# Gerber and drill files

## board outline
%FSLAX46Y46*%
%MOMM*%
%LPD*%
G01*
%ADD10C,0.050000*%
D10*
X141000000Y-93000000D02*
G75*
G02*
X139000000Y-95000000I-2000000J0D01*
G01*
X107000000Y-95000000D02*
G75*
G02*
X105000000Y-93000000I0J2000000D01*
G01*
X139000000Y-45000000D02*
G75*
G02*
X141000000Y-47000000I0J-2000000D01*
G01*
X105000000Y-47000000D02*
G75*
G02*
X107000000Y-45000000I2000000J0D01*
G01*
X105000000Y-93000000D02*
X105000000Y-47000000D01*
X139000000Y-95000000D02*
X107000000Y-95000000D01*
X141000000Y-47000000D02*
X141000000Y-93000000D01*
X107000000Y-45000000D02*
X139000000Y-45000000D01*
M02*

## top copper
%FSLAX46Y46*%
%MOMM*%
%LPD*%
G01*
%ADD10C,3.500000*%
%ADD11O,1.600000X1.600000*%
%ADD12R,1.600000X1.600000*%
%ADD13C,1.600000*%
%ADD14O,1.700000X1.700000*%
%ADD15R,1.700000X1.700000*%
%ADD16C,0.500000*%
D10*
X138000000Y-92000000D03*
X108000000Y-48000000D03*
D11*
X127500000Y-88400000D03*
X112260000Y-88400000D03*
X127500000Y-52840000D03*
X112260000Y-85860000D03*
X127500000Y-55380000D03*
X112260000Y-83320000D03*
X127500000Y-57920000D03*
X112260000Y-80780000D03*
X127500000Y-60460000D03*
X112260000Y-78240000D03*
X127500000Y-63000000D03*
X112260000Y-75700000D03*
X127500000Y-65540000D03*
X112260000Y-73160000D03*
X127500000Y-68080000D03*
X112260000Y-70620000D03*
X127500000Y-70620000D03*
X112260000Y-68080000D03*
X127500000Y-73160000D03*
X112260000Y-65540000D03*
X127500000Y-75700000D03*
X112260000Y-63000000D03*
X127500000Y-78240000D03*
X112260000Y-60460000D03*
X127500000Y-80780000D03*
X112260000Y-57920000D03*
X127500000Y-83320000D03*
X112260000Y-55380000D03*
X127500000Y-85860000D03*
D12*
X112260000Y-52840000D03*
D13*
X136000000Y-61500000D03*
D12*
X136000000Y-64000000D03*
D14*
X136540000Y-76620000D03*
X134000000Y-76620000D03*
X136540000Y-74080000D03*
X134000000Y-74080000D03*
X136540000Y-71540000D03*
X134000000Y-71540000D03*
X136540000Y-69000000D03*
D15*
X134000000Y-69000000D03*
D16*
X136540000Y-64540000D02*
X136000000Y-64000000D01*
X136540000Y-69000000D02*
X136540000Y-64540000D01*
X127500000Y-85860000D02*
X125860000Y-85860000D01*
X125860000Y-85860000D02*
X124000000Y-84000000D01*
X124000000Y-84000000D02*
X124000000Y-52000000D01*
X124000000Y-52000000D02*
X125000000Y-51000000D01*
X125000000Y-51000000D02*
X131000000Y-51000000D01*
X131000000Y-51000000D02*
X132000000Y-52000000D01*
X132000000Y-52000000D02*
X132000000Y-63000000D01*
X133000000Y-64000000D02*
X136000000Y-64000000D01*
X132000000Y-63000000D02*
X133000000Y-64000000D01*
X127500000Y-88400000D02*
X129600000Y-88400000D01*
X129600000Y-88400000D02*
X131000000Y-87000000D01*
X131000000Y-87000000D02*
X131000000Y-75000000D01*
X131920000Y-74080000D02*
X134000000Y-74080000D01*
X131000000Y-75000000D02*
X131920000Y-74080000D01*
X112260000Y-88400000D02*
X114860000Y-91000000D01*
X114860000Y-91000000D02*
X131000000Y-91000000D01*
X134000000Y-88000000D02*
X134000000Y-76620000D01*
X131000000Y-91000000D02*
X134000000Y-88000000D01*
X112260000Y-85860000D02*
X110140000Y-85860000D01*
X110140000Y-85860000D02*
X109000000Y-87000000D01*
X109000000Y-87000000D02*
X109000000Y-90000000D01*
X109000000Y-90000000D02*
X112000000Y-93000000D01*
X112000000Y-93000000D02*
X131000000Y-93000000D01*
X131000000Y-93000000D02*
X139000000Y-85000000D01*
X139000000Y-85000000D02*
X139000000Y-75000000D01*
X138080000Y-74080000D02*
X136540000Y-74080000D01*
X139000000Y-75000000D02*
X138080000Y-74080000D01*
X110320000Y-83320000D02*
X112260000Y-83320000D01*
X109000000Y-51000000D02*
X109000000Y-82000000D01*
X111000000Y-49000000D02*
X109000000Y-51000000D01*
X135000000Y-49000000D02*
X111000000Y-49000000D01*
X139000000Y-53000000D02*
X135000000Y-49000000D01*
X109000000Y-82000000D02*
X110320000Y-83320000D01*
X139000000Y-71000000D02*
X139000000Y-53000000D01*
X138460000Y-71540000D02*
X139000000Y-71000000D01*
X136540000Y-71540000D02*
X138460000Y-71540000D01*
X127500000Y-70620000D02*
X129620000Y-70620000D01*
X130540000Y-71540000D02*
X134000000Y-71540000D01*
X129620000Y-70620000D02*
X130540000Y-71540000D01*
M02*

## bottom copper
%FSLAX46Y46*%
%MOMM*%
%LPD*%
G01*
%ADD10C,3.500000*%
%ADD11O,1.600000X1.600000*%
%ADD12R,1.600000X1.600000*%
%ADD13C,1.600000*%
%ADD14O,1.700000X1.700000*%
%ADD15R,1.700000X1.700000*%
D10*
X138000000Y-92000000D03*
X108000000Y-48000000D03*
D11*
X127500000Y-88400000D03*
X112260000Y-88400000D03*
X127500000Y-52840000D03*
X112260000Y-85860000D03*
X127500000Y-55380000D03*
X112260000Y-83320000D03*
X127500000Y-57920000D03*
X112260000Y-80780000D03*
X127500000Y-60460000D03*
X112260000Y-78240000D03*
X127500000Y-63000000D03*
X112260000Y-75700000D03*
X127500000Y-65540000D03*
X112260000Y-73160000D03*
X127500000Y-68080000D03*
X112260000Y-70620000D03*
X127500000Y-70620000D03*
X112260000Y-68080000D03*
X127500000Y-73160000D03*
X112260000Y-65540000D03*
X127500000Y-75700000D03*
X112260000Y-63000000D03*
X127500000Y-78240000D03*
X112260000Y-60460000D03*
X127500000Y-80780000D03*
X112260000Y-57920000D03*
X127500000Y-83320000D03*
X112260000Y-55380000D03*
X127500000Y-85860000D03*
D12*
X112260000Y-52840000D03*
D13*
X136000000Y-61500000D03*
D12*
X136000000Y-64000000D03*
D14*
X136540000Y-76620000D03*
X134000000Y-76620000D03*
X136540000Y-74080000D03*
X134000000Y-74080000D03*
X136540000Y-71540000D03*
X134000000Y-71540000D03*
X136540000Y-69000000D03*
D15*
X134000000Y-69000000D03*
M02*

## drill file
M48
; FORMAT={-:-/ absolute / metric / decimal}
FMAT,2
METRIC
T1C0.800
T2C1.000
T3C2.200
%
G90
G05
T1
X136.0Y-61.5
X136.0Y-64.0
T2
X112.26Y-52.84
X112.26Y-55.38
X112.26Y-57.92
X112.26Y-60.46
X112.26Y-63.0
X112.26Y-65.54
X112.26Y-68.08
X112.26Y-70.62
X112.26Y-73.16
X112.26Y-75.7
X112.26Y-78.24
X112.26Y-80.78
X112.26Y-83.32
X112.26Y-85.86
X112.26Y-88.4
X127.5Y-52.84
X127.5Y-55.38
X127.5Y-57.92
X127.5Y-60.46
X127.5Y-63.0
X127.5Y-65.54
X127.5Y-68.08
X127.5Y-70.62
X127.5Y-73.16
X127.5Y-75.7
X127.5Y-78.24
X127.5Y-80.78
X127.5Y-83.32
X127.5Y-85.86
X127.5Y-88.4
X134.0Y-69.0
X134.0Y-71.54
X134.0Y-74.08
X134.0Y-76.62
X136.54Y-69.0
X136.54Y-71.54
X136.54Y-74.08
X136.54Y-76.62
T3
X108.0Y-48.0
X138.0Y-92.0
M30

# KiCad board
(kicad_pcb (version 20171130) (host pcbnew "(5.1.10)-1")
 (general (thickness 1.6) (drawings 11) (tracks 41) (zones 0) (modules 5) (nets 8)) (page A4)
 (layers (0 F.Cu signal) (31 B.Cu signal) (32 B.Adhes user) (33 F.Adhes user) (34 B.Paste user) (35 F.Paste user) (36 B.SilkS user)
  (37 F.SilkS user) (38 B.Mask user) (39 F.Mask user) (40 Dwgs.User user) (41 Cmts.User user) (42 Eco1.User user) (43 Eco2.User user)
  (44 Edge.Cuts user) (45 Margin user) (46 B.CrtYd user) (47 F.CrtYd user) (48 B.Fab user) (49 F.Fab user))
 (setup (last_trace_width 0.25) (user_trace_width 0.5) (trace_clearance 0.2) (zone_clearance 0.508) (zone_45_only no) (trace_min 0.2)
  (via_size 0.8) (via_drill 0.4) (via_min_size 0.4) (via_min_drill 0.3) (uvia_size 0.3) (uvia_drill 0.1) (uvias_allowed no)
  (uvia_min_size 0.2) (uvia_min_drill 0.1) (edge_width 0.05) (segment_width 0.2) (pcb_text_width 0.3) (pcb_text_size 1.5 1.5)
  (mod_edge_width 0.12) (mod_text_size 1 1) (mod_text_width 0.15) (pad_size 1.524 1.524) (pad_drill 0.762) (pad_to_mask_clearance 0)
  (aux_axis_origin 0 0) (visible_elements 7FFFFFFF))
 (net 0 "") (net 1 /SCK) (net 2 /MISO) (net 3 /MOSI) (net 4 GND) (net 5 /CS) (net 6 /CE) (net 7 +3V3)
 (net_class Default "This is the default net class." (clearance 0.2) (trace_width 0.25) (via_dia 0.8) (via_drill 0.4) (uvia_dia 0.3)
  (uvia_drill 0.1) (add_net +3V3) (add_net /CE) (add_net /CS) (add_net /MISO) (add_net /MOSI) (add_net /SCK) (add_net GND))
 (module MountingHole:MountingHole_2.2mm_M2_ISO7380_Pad (layer F.Cu) (at 138 92)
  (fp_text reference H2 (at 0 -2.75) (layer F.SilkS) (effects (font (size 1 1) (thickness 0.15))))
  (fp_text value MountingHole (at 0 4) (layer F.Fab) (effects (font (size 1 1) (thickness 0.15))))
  (pad 1 thru_hole circle (at 0 0) (size 3.5 3.5) (drill 2.2) (layers *.Cu *.Mask)))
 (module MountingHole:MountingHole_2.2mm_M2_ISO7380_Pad (layer F.Cu) (at 108 48)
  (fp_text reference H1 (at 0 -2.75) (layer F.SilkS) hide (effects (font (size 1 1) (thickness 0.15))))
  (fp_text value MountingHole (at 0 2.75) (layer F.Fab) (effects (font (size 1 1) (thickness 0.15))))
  (pad 1 thru_hole circle (at 0 0) (size 3.5 3.5) (drill 2.2) (layers *.Cu *.Mask)))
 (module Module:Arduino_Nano (layer F.Cu) (at 112.26 52.84)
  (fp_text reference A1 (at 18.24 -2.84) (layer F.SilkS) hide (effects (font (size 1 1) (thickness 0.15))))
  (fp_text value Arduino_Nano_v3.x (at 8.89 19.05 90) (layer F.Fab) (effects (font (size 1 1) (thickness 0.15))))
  (pad 16 thru_hole oval (at 15.24 35.56) (size 1.6 1.6) (drill 1) (layers *.Cu *.Mask) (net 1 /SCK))
  (pad 15 thru_hole oval (at 0 35.56) (size 1.6 1.6) (drill 1) (layers *.Cu *.Mask) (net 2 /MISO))
  (pad 30 thru_hole oval (at 15.24 0) (size 1.6 1.6) (drill 1) (layers *.Cu *.Mask))
  (pad 14 thru_hole oval (at 0 33.02) (size 1.6 1.6) (drill 1) (layers *.Cu *.Mask) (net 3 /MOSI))
  (pad 29 thru_hole oval (at 15.24 2.54) (size 1.6 1.6) (drill 1) (layers *.Cu *.Mask) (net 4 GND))
  (pad 13 thru_hole oval (at 0 30.48) (size 1.6 1.6) (drill 1) (layers *.Cu *.Mask) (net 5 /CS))
  (pad 28 thru_hole oval (at 15.24 5.08) (size 1.6 1.6) (drill 1) (layers *.Cu *.Mask))
  (pad 12 thru_hole oval (at 0 27.94) (size 1.6 1.6) (drill 1) (layers *.Cu *.Mask))
  (pad 27 thru_hole oval (at 15.24 7.62) (size 1.6 1.6) (drill 1) (layers *.Cu *.Mask))
  (pad 11 thru_hole oval (at 0 25.4) (size 1.6 1.6) (drill 1) (layers *.Cu *.Mask))
  (pad 26 thru_hole oval (at 15.24 10.16) (size 1.6 1.6) (drill 1) (layers *.Cu *.Mask))
  (pad 10 thru_hole oval (at 0 22.86) (size 1.6 1.6) (drill 1) (layers *.Cu *.Mask))
  (pad 25 thru_hole oval (at 15.24 12.7) (size 1.6 1.6) (drill 1) (layers *.Cu *.Mask))
  (pad 9 thru_hole oval (at 0 20.32) (size 1.6 1.6) (drill 1) (layers *.Cu *.Mask))
  (pad 24 thru_hole oval (at 15.24 15.24) (size 1.6 1.6) (drill 1) (layers *.Cu *.Mask))
  (pad 8 thru_hole oval (at 0 17.78) (size 1.6 1.6) (drill 1) (layers *.Cu *.Mask))
  (pad 23 thru_hole oval (at 15.24 17.78) (size 1.6 1.6) (drill 1) (layers *.Cu *.Mask) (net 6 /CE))
  (pad 7 thru_hole oval (at 0 15.24) (size 1.6 1.6) (drill 1) (layers *.Cu *.Mask))
  (pad 22 thru_hole oval (at 15.24 20.32) (size 1.6 1.6) (drill 1) (layers *.Cu *.Mask))
  (pad 6 thru_hole oval (at 0 12.7) (size 1.6 1.6) (drill 1) (layers *.Cu *.Mask))
  (pad 21 thru_hole oval (at 15.24 22.86) (size 1.6 1.6) (drill 1) (layers *.Cu *.Mask))
  (pad 5 thru_hole oval (at 0 10.16) (size 1.6 1.6) (drill 1) (layers *.Cu *.Mask))
  (pad 20 thru_hole oval (at 15.24 25.4) (size 1.6 1.6) (drill 1) (layers *.Cu *.Mask))
  (pad 4 thru_hole oval (at 0 7.62) (size 1.6 1.6) (drill 1) (layers *.Cu *.Mask) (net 4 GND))
  (pad 19 thru_hole oval (at 15.24 27.94) (size 1.6 1.6) (drill 1) (layers *.Cu *.Mask))
  (pad 3 thru_hole oval (at 0 5.08) (size 1.6 1.6) (drill 1) (layers *.Cu *.Mask))
  (pad 18 thru_hole oval (at 15.24 30.48) (size 1.6 1.6) (drill 1) (layers *.Cu *.Mask))
  (pad 2 thru_hole oval (at 0 2.54) (size 1.6 1.6) (drill 1) (layers *.Cu *.Mask))
  (pad 17 thru_hole oval (at 15.24 33.02) (size 1.6 1.6) (drill 1) (layers *.Cu *.Mask) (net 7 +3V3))
  (pad 1 thru_hole rect (at 0 0) (size 1.6 1.6) (drill 1) (layers *.Cu *.Mask)))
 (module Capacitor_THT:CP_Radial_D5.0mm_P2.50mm (layer F.Cu) (at 136 64 90)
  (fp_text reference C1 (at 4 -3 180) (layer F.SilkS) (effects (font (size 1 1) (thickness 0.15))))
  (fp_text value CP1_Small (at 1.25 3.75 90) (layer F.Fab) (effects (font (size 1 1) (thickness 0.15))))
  (pad 2 thru_hole circle (at 2.5 0 90) (size 1.6 1.6) (drill 0.8) (layers *.Cu *.Mask) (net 4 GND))
  (pad 1 thru_hole rect (at 0 0 90) (size 1.6 1.6) (drill 0.8) (layers *.Cu *.Mask) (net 7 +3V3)))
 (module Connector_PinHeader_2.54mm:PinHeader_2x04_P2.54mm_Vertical (layer F.Cu) (at 134 69)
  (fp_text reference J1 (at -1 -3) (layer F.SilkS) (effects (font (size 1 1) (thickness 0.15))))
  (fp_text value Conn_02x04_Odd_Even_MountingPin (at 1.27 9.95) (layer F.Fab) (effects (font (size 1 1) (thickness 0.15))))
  (pad 8 thru_hole oval (at 2.54 7.62) (size 1.7 1.7) (drill 1) (layers *.Cu *.Mask))
  (pad 7 thru_hole oval (at 0 7.62) (size 1.7 1.7) (drill 1) (layers *.Cu *.Mask) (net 2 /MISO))
  (pad 6 thru_hole oval (at 2.54 5.08) (size 1.7 1.7) (drill 1) (layers *.Cu *.Mask) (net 3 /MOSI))
  (pad 5 thru_hole oval (at 0 5.08) (size 1.7 1.7) (drill 1) (layers *.Cu *.Mask) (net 1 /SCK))
  (pad 4 thru_hole oval (at 2.54 2.54) (size 1.7 1.7) (drill 1) (layers *.Cu *.Mask) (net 5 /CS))
  (pad 3 thru_hole oval (at 0 2.54) (size 1.7 1.7) (drill 1) (layers *.Cu *.Mask) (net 6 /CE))
  (pad 2 thru_hole oval (at 2.54 0) (size 1.7 1.7) (drill 1) (layers *.Cu *.Mask) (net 7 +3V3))
  (pad 1 thru_hole rect (at 0 0) (size 1.7 1.7) (drill 1) (layers *.Cu *.Mask) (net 4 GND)))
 (gr_arc (start 139 93) (end 139 95) (angle -90) (layer Edge.Cuts) (width 0.05))
 (gr_arc (start 107 93) (end 105 93) (angle -90) (layer Edge.Cuts) (width 0.05))
 (gr_arc (start 139 47) (end 141 47) (angle -90) (layer Edge.Cuts) (width 0.05))
 (gr_arc (start 107 47) (end 107 45) (angle -90) (layer Edge.Cuts) (width 0.05))
 (gr_line (start 105 93) (end 105 47) (layer Edge.Cuts) (width 0.05))
 (gr_line (start 139 95) (end 107 95) (layer Edge.Cuts) (width 0.05))
 (gr_line (start 141 47) (end 141 93) (layer Edge.Cuts) (width 0.05))
 (gr_line (start 107 45) (end 139 45) (layer Edge.Cuts) (width 0.05))
 (segment (start 136.54 64.54) (end 136 64) (width 0.5) (layer F.Cu) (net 7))
 (segment (start 136.54 69) (end 136.54 64.54) (width 0.5) (layer F.Cu) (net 7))
 (segment (start 127.5 85.86) (end 125.86 85.86) (width 0.5) (layer F.Cu) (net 7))
 (segment (start 125.86 85.86) (end 124 84) (width 0.5) (layer F.Cu) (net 7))
 (segment (start 124 84) (end 124 52) (width 0.5) (layer F.Cu) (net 7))
 (segment (start 124 52) (end 125 51) (width 0.5) (layer F.Cu) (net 7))
 (segment (start 125 51) (end 131 51) (width 0.5) (layer F.Cu) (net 7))
 (segment (start 131 51) (end 132 52) (width 0.5) (layer F.Cu) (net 7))
 (segment (start 132 52) (end 132 63) (width 0.5) (layer F.Cu) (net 7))
 (segment (start 133 64) (end 136 64) (width 0.5) (layer F.Cu) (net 7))
 (segment (start 132 63) (end 133 64) (width 0.5) (layer F.Cu) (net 7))
 (segment (start 127.5 88.4) (end 129.6 88.4) (width 0.5) (layer F.Cu) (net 1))
 (segment (start 129.6 88.4) (end 131 87) (width 0.5) (layer F.Cu) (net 1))
 (segment (start 131 87) (end 131 75) (width 0.5) (layer F.Cu) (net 1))
 (segment (start 131.92 74.08) (end 134 74.08) (width 0.5) (layer F.Cu) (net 1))
 (segment (start 131 75) (end 131.92 74.08) (width 0.5) (layer F.Cu) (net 1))
 (segment (start 112.26 88.4) (end 114.86 91) (width 0.5) (layer F.Cu) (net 2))
 (segment (start 114.86 91) (end 131 91) (width 0.5) (layer F.Cu) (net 2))
 (segment (start 134 88) (end 134 76.62) (width 0.5) (layer F.Cu) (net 2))
 (segment (start 131 91) (end 134 88) (width 0.5) (layer F.Cu) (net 2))
 (segment (start 112.26 85.86) (end 110.14 85.86) (width 0.5) (layer F.Cu) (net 3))
 (segment (start 110.14 85.86) (end 109 87) (width 0.5) (layer F.Cu) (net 3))
 (segment (start 109 87) (end 109 90) (width 0.5) (layer F.Cu) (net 3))
 (segment (start 109 90) (end 112 93) (width 0.5) (layer F.Cu) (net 3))
 (segment (start 112 93) (end 131 93) (width 0.5) (layer F.Cu) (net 3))
 (segment (start 131 93) (end 139 85) (width 0.5) (layer F.Cu) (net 3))
 (segment (start 139 85) (end 139 75) (width 0.5) (layer F.Cu) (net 3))
 (segment (start 138.08 74.08) (end 136.54 74.08) (width 0.5) (layer F.Cu) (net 3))
 (segment (start 139 75) (end 138.08 74.08) (width 0.5) (layer F.Cu) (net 3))
 (segment (start 110.32 83.32) (end 112.26 83.32) (width 0.5) (layer F.Cu) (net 5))
 (segment (start 109 51) (end 109 82) (width 0.5) (layer F.Cu) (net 5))
 (segment (start 111 49) (end 109 51) (width 0.5) (layer F.Cu) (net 5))
 (segment (start 135 49) (end 111 49) (width 0.5) (layer F.Cu) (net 5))
 (segment (start 139 53) (end 135 49) (width 0.5) (layer F.Cu) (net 5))
 (segment (start 109 82) (end 110.32 83.32) (width 0.5) (layer F.Cu) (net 5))
 (segment (start 139 71) (end 139 53) (width 0.5) (layer F.Cu) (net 5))
 (segment (start 138.46 71.54) (end 139 71) (width 0.5) (layer F.Cu) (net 5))
 (segment (start 136.54 71.54) (end 138.46 71.54) (width 0.5) (layer F.Cu) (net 5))
 (segment (start 127.5 70.62) (end 129.62 70.62) (width 0.5) (layer F.Cu) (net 6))
 (segment (start 130.54 71.54) (end 134 71.54) (width 0.5) (layer F.Cu) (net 6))
 (segment (start 129.62 70.62) (end 130.54 71.54) (width 0.5) (layer F.Cu) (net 6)))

